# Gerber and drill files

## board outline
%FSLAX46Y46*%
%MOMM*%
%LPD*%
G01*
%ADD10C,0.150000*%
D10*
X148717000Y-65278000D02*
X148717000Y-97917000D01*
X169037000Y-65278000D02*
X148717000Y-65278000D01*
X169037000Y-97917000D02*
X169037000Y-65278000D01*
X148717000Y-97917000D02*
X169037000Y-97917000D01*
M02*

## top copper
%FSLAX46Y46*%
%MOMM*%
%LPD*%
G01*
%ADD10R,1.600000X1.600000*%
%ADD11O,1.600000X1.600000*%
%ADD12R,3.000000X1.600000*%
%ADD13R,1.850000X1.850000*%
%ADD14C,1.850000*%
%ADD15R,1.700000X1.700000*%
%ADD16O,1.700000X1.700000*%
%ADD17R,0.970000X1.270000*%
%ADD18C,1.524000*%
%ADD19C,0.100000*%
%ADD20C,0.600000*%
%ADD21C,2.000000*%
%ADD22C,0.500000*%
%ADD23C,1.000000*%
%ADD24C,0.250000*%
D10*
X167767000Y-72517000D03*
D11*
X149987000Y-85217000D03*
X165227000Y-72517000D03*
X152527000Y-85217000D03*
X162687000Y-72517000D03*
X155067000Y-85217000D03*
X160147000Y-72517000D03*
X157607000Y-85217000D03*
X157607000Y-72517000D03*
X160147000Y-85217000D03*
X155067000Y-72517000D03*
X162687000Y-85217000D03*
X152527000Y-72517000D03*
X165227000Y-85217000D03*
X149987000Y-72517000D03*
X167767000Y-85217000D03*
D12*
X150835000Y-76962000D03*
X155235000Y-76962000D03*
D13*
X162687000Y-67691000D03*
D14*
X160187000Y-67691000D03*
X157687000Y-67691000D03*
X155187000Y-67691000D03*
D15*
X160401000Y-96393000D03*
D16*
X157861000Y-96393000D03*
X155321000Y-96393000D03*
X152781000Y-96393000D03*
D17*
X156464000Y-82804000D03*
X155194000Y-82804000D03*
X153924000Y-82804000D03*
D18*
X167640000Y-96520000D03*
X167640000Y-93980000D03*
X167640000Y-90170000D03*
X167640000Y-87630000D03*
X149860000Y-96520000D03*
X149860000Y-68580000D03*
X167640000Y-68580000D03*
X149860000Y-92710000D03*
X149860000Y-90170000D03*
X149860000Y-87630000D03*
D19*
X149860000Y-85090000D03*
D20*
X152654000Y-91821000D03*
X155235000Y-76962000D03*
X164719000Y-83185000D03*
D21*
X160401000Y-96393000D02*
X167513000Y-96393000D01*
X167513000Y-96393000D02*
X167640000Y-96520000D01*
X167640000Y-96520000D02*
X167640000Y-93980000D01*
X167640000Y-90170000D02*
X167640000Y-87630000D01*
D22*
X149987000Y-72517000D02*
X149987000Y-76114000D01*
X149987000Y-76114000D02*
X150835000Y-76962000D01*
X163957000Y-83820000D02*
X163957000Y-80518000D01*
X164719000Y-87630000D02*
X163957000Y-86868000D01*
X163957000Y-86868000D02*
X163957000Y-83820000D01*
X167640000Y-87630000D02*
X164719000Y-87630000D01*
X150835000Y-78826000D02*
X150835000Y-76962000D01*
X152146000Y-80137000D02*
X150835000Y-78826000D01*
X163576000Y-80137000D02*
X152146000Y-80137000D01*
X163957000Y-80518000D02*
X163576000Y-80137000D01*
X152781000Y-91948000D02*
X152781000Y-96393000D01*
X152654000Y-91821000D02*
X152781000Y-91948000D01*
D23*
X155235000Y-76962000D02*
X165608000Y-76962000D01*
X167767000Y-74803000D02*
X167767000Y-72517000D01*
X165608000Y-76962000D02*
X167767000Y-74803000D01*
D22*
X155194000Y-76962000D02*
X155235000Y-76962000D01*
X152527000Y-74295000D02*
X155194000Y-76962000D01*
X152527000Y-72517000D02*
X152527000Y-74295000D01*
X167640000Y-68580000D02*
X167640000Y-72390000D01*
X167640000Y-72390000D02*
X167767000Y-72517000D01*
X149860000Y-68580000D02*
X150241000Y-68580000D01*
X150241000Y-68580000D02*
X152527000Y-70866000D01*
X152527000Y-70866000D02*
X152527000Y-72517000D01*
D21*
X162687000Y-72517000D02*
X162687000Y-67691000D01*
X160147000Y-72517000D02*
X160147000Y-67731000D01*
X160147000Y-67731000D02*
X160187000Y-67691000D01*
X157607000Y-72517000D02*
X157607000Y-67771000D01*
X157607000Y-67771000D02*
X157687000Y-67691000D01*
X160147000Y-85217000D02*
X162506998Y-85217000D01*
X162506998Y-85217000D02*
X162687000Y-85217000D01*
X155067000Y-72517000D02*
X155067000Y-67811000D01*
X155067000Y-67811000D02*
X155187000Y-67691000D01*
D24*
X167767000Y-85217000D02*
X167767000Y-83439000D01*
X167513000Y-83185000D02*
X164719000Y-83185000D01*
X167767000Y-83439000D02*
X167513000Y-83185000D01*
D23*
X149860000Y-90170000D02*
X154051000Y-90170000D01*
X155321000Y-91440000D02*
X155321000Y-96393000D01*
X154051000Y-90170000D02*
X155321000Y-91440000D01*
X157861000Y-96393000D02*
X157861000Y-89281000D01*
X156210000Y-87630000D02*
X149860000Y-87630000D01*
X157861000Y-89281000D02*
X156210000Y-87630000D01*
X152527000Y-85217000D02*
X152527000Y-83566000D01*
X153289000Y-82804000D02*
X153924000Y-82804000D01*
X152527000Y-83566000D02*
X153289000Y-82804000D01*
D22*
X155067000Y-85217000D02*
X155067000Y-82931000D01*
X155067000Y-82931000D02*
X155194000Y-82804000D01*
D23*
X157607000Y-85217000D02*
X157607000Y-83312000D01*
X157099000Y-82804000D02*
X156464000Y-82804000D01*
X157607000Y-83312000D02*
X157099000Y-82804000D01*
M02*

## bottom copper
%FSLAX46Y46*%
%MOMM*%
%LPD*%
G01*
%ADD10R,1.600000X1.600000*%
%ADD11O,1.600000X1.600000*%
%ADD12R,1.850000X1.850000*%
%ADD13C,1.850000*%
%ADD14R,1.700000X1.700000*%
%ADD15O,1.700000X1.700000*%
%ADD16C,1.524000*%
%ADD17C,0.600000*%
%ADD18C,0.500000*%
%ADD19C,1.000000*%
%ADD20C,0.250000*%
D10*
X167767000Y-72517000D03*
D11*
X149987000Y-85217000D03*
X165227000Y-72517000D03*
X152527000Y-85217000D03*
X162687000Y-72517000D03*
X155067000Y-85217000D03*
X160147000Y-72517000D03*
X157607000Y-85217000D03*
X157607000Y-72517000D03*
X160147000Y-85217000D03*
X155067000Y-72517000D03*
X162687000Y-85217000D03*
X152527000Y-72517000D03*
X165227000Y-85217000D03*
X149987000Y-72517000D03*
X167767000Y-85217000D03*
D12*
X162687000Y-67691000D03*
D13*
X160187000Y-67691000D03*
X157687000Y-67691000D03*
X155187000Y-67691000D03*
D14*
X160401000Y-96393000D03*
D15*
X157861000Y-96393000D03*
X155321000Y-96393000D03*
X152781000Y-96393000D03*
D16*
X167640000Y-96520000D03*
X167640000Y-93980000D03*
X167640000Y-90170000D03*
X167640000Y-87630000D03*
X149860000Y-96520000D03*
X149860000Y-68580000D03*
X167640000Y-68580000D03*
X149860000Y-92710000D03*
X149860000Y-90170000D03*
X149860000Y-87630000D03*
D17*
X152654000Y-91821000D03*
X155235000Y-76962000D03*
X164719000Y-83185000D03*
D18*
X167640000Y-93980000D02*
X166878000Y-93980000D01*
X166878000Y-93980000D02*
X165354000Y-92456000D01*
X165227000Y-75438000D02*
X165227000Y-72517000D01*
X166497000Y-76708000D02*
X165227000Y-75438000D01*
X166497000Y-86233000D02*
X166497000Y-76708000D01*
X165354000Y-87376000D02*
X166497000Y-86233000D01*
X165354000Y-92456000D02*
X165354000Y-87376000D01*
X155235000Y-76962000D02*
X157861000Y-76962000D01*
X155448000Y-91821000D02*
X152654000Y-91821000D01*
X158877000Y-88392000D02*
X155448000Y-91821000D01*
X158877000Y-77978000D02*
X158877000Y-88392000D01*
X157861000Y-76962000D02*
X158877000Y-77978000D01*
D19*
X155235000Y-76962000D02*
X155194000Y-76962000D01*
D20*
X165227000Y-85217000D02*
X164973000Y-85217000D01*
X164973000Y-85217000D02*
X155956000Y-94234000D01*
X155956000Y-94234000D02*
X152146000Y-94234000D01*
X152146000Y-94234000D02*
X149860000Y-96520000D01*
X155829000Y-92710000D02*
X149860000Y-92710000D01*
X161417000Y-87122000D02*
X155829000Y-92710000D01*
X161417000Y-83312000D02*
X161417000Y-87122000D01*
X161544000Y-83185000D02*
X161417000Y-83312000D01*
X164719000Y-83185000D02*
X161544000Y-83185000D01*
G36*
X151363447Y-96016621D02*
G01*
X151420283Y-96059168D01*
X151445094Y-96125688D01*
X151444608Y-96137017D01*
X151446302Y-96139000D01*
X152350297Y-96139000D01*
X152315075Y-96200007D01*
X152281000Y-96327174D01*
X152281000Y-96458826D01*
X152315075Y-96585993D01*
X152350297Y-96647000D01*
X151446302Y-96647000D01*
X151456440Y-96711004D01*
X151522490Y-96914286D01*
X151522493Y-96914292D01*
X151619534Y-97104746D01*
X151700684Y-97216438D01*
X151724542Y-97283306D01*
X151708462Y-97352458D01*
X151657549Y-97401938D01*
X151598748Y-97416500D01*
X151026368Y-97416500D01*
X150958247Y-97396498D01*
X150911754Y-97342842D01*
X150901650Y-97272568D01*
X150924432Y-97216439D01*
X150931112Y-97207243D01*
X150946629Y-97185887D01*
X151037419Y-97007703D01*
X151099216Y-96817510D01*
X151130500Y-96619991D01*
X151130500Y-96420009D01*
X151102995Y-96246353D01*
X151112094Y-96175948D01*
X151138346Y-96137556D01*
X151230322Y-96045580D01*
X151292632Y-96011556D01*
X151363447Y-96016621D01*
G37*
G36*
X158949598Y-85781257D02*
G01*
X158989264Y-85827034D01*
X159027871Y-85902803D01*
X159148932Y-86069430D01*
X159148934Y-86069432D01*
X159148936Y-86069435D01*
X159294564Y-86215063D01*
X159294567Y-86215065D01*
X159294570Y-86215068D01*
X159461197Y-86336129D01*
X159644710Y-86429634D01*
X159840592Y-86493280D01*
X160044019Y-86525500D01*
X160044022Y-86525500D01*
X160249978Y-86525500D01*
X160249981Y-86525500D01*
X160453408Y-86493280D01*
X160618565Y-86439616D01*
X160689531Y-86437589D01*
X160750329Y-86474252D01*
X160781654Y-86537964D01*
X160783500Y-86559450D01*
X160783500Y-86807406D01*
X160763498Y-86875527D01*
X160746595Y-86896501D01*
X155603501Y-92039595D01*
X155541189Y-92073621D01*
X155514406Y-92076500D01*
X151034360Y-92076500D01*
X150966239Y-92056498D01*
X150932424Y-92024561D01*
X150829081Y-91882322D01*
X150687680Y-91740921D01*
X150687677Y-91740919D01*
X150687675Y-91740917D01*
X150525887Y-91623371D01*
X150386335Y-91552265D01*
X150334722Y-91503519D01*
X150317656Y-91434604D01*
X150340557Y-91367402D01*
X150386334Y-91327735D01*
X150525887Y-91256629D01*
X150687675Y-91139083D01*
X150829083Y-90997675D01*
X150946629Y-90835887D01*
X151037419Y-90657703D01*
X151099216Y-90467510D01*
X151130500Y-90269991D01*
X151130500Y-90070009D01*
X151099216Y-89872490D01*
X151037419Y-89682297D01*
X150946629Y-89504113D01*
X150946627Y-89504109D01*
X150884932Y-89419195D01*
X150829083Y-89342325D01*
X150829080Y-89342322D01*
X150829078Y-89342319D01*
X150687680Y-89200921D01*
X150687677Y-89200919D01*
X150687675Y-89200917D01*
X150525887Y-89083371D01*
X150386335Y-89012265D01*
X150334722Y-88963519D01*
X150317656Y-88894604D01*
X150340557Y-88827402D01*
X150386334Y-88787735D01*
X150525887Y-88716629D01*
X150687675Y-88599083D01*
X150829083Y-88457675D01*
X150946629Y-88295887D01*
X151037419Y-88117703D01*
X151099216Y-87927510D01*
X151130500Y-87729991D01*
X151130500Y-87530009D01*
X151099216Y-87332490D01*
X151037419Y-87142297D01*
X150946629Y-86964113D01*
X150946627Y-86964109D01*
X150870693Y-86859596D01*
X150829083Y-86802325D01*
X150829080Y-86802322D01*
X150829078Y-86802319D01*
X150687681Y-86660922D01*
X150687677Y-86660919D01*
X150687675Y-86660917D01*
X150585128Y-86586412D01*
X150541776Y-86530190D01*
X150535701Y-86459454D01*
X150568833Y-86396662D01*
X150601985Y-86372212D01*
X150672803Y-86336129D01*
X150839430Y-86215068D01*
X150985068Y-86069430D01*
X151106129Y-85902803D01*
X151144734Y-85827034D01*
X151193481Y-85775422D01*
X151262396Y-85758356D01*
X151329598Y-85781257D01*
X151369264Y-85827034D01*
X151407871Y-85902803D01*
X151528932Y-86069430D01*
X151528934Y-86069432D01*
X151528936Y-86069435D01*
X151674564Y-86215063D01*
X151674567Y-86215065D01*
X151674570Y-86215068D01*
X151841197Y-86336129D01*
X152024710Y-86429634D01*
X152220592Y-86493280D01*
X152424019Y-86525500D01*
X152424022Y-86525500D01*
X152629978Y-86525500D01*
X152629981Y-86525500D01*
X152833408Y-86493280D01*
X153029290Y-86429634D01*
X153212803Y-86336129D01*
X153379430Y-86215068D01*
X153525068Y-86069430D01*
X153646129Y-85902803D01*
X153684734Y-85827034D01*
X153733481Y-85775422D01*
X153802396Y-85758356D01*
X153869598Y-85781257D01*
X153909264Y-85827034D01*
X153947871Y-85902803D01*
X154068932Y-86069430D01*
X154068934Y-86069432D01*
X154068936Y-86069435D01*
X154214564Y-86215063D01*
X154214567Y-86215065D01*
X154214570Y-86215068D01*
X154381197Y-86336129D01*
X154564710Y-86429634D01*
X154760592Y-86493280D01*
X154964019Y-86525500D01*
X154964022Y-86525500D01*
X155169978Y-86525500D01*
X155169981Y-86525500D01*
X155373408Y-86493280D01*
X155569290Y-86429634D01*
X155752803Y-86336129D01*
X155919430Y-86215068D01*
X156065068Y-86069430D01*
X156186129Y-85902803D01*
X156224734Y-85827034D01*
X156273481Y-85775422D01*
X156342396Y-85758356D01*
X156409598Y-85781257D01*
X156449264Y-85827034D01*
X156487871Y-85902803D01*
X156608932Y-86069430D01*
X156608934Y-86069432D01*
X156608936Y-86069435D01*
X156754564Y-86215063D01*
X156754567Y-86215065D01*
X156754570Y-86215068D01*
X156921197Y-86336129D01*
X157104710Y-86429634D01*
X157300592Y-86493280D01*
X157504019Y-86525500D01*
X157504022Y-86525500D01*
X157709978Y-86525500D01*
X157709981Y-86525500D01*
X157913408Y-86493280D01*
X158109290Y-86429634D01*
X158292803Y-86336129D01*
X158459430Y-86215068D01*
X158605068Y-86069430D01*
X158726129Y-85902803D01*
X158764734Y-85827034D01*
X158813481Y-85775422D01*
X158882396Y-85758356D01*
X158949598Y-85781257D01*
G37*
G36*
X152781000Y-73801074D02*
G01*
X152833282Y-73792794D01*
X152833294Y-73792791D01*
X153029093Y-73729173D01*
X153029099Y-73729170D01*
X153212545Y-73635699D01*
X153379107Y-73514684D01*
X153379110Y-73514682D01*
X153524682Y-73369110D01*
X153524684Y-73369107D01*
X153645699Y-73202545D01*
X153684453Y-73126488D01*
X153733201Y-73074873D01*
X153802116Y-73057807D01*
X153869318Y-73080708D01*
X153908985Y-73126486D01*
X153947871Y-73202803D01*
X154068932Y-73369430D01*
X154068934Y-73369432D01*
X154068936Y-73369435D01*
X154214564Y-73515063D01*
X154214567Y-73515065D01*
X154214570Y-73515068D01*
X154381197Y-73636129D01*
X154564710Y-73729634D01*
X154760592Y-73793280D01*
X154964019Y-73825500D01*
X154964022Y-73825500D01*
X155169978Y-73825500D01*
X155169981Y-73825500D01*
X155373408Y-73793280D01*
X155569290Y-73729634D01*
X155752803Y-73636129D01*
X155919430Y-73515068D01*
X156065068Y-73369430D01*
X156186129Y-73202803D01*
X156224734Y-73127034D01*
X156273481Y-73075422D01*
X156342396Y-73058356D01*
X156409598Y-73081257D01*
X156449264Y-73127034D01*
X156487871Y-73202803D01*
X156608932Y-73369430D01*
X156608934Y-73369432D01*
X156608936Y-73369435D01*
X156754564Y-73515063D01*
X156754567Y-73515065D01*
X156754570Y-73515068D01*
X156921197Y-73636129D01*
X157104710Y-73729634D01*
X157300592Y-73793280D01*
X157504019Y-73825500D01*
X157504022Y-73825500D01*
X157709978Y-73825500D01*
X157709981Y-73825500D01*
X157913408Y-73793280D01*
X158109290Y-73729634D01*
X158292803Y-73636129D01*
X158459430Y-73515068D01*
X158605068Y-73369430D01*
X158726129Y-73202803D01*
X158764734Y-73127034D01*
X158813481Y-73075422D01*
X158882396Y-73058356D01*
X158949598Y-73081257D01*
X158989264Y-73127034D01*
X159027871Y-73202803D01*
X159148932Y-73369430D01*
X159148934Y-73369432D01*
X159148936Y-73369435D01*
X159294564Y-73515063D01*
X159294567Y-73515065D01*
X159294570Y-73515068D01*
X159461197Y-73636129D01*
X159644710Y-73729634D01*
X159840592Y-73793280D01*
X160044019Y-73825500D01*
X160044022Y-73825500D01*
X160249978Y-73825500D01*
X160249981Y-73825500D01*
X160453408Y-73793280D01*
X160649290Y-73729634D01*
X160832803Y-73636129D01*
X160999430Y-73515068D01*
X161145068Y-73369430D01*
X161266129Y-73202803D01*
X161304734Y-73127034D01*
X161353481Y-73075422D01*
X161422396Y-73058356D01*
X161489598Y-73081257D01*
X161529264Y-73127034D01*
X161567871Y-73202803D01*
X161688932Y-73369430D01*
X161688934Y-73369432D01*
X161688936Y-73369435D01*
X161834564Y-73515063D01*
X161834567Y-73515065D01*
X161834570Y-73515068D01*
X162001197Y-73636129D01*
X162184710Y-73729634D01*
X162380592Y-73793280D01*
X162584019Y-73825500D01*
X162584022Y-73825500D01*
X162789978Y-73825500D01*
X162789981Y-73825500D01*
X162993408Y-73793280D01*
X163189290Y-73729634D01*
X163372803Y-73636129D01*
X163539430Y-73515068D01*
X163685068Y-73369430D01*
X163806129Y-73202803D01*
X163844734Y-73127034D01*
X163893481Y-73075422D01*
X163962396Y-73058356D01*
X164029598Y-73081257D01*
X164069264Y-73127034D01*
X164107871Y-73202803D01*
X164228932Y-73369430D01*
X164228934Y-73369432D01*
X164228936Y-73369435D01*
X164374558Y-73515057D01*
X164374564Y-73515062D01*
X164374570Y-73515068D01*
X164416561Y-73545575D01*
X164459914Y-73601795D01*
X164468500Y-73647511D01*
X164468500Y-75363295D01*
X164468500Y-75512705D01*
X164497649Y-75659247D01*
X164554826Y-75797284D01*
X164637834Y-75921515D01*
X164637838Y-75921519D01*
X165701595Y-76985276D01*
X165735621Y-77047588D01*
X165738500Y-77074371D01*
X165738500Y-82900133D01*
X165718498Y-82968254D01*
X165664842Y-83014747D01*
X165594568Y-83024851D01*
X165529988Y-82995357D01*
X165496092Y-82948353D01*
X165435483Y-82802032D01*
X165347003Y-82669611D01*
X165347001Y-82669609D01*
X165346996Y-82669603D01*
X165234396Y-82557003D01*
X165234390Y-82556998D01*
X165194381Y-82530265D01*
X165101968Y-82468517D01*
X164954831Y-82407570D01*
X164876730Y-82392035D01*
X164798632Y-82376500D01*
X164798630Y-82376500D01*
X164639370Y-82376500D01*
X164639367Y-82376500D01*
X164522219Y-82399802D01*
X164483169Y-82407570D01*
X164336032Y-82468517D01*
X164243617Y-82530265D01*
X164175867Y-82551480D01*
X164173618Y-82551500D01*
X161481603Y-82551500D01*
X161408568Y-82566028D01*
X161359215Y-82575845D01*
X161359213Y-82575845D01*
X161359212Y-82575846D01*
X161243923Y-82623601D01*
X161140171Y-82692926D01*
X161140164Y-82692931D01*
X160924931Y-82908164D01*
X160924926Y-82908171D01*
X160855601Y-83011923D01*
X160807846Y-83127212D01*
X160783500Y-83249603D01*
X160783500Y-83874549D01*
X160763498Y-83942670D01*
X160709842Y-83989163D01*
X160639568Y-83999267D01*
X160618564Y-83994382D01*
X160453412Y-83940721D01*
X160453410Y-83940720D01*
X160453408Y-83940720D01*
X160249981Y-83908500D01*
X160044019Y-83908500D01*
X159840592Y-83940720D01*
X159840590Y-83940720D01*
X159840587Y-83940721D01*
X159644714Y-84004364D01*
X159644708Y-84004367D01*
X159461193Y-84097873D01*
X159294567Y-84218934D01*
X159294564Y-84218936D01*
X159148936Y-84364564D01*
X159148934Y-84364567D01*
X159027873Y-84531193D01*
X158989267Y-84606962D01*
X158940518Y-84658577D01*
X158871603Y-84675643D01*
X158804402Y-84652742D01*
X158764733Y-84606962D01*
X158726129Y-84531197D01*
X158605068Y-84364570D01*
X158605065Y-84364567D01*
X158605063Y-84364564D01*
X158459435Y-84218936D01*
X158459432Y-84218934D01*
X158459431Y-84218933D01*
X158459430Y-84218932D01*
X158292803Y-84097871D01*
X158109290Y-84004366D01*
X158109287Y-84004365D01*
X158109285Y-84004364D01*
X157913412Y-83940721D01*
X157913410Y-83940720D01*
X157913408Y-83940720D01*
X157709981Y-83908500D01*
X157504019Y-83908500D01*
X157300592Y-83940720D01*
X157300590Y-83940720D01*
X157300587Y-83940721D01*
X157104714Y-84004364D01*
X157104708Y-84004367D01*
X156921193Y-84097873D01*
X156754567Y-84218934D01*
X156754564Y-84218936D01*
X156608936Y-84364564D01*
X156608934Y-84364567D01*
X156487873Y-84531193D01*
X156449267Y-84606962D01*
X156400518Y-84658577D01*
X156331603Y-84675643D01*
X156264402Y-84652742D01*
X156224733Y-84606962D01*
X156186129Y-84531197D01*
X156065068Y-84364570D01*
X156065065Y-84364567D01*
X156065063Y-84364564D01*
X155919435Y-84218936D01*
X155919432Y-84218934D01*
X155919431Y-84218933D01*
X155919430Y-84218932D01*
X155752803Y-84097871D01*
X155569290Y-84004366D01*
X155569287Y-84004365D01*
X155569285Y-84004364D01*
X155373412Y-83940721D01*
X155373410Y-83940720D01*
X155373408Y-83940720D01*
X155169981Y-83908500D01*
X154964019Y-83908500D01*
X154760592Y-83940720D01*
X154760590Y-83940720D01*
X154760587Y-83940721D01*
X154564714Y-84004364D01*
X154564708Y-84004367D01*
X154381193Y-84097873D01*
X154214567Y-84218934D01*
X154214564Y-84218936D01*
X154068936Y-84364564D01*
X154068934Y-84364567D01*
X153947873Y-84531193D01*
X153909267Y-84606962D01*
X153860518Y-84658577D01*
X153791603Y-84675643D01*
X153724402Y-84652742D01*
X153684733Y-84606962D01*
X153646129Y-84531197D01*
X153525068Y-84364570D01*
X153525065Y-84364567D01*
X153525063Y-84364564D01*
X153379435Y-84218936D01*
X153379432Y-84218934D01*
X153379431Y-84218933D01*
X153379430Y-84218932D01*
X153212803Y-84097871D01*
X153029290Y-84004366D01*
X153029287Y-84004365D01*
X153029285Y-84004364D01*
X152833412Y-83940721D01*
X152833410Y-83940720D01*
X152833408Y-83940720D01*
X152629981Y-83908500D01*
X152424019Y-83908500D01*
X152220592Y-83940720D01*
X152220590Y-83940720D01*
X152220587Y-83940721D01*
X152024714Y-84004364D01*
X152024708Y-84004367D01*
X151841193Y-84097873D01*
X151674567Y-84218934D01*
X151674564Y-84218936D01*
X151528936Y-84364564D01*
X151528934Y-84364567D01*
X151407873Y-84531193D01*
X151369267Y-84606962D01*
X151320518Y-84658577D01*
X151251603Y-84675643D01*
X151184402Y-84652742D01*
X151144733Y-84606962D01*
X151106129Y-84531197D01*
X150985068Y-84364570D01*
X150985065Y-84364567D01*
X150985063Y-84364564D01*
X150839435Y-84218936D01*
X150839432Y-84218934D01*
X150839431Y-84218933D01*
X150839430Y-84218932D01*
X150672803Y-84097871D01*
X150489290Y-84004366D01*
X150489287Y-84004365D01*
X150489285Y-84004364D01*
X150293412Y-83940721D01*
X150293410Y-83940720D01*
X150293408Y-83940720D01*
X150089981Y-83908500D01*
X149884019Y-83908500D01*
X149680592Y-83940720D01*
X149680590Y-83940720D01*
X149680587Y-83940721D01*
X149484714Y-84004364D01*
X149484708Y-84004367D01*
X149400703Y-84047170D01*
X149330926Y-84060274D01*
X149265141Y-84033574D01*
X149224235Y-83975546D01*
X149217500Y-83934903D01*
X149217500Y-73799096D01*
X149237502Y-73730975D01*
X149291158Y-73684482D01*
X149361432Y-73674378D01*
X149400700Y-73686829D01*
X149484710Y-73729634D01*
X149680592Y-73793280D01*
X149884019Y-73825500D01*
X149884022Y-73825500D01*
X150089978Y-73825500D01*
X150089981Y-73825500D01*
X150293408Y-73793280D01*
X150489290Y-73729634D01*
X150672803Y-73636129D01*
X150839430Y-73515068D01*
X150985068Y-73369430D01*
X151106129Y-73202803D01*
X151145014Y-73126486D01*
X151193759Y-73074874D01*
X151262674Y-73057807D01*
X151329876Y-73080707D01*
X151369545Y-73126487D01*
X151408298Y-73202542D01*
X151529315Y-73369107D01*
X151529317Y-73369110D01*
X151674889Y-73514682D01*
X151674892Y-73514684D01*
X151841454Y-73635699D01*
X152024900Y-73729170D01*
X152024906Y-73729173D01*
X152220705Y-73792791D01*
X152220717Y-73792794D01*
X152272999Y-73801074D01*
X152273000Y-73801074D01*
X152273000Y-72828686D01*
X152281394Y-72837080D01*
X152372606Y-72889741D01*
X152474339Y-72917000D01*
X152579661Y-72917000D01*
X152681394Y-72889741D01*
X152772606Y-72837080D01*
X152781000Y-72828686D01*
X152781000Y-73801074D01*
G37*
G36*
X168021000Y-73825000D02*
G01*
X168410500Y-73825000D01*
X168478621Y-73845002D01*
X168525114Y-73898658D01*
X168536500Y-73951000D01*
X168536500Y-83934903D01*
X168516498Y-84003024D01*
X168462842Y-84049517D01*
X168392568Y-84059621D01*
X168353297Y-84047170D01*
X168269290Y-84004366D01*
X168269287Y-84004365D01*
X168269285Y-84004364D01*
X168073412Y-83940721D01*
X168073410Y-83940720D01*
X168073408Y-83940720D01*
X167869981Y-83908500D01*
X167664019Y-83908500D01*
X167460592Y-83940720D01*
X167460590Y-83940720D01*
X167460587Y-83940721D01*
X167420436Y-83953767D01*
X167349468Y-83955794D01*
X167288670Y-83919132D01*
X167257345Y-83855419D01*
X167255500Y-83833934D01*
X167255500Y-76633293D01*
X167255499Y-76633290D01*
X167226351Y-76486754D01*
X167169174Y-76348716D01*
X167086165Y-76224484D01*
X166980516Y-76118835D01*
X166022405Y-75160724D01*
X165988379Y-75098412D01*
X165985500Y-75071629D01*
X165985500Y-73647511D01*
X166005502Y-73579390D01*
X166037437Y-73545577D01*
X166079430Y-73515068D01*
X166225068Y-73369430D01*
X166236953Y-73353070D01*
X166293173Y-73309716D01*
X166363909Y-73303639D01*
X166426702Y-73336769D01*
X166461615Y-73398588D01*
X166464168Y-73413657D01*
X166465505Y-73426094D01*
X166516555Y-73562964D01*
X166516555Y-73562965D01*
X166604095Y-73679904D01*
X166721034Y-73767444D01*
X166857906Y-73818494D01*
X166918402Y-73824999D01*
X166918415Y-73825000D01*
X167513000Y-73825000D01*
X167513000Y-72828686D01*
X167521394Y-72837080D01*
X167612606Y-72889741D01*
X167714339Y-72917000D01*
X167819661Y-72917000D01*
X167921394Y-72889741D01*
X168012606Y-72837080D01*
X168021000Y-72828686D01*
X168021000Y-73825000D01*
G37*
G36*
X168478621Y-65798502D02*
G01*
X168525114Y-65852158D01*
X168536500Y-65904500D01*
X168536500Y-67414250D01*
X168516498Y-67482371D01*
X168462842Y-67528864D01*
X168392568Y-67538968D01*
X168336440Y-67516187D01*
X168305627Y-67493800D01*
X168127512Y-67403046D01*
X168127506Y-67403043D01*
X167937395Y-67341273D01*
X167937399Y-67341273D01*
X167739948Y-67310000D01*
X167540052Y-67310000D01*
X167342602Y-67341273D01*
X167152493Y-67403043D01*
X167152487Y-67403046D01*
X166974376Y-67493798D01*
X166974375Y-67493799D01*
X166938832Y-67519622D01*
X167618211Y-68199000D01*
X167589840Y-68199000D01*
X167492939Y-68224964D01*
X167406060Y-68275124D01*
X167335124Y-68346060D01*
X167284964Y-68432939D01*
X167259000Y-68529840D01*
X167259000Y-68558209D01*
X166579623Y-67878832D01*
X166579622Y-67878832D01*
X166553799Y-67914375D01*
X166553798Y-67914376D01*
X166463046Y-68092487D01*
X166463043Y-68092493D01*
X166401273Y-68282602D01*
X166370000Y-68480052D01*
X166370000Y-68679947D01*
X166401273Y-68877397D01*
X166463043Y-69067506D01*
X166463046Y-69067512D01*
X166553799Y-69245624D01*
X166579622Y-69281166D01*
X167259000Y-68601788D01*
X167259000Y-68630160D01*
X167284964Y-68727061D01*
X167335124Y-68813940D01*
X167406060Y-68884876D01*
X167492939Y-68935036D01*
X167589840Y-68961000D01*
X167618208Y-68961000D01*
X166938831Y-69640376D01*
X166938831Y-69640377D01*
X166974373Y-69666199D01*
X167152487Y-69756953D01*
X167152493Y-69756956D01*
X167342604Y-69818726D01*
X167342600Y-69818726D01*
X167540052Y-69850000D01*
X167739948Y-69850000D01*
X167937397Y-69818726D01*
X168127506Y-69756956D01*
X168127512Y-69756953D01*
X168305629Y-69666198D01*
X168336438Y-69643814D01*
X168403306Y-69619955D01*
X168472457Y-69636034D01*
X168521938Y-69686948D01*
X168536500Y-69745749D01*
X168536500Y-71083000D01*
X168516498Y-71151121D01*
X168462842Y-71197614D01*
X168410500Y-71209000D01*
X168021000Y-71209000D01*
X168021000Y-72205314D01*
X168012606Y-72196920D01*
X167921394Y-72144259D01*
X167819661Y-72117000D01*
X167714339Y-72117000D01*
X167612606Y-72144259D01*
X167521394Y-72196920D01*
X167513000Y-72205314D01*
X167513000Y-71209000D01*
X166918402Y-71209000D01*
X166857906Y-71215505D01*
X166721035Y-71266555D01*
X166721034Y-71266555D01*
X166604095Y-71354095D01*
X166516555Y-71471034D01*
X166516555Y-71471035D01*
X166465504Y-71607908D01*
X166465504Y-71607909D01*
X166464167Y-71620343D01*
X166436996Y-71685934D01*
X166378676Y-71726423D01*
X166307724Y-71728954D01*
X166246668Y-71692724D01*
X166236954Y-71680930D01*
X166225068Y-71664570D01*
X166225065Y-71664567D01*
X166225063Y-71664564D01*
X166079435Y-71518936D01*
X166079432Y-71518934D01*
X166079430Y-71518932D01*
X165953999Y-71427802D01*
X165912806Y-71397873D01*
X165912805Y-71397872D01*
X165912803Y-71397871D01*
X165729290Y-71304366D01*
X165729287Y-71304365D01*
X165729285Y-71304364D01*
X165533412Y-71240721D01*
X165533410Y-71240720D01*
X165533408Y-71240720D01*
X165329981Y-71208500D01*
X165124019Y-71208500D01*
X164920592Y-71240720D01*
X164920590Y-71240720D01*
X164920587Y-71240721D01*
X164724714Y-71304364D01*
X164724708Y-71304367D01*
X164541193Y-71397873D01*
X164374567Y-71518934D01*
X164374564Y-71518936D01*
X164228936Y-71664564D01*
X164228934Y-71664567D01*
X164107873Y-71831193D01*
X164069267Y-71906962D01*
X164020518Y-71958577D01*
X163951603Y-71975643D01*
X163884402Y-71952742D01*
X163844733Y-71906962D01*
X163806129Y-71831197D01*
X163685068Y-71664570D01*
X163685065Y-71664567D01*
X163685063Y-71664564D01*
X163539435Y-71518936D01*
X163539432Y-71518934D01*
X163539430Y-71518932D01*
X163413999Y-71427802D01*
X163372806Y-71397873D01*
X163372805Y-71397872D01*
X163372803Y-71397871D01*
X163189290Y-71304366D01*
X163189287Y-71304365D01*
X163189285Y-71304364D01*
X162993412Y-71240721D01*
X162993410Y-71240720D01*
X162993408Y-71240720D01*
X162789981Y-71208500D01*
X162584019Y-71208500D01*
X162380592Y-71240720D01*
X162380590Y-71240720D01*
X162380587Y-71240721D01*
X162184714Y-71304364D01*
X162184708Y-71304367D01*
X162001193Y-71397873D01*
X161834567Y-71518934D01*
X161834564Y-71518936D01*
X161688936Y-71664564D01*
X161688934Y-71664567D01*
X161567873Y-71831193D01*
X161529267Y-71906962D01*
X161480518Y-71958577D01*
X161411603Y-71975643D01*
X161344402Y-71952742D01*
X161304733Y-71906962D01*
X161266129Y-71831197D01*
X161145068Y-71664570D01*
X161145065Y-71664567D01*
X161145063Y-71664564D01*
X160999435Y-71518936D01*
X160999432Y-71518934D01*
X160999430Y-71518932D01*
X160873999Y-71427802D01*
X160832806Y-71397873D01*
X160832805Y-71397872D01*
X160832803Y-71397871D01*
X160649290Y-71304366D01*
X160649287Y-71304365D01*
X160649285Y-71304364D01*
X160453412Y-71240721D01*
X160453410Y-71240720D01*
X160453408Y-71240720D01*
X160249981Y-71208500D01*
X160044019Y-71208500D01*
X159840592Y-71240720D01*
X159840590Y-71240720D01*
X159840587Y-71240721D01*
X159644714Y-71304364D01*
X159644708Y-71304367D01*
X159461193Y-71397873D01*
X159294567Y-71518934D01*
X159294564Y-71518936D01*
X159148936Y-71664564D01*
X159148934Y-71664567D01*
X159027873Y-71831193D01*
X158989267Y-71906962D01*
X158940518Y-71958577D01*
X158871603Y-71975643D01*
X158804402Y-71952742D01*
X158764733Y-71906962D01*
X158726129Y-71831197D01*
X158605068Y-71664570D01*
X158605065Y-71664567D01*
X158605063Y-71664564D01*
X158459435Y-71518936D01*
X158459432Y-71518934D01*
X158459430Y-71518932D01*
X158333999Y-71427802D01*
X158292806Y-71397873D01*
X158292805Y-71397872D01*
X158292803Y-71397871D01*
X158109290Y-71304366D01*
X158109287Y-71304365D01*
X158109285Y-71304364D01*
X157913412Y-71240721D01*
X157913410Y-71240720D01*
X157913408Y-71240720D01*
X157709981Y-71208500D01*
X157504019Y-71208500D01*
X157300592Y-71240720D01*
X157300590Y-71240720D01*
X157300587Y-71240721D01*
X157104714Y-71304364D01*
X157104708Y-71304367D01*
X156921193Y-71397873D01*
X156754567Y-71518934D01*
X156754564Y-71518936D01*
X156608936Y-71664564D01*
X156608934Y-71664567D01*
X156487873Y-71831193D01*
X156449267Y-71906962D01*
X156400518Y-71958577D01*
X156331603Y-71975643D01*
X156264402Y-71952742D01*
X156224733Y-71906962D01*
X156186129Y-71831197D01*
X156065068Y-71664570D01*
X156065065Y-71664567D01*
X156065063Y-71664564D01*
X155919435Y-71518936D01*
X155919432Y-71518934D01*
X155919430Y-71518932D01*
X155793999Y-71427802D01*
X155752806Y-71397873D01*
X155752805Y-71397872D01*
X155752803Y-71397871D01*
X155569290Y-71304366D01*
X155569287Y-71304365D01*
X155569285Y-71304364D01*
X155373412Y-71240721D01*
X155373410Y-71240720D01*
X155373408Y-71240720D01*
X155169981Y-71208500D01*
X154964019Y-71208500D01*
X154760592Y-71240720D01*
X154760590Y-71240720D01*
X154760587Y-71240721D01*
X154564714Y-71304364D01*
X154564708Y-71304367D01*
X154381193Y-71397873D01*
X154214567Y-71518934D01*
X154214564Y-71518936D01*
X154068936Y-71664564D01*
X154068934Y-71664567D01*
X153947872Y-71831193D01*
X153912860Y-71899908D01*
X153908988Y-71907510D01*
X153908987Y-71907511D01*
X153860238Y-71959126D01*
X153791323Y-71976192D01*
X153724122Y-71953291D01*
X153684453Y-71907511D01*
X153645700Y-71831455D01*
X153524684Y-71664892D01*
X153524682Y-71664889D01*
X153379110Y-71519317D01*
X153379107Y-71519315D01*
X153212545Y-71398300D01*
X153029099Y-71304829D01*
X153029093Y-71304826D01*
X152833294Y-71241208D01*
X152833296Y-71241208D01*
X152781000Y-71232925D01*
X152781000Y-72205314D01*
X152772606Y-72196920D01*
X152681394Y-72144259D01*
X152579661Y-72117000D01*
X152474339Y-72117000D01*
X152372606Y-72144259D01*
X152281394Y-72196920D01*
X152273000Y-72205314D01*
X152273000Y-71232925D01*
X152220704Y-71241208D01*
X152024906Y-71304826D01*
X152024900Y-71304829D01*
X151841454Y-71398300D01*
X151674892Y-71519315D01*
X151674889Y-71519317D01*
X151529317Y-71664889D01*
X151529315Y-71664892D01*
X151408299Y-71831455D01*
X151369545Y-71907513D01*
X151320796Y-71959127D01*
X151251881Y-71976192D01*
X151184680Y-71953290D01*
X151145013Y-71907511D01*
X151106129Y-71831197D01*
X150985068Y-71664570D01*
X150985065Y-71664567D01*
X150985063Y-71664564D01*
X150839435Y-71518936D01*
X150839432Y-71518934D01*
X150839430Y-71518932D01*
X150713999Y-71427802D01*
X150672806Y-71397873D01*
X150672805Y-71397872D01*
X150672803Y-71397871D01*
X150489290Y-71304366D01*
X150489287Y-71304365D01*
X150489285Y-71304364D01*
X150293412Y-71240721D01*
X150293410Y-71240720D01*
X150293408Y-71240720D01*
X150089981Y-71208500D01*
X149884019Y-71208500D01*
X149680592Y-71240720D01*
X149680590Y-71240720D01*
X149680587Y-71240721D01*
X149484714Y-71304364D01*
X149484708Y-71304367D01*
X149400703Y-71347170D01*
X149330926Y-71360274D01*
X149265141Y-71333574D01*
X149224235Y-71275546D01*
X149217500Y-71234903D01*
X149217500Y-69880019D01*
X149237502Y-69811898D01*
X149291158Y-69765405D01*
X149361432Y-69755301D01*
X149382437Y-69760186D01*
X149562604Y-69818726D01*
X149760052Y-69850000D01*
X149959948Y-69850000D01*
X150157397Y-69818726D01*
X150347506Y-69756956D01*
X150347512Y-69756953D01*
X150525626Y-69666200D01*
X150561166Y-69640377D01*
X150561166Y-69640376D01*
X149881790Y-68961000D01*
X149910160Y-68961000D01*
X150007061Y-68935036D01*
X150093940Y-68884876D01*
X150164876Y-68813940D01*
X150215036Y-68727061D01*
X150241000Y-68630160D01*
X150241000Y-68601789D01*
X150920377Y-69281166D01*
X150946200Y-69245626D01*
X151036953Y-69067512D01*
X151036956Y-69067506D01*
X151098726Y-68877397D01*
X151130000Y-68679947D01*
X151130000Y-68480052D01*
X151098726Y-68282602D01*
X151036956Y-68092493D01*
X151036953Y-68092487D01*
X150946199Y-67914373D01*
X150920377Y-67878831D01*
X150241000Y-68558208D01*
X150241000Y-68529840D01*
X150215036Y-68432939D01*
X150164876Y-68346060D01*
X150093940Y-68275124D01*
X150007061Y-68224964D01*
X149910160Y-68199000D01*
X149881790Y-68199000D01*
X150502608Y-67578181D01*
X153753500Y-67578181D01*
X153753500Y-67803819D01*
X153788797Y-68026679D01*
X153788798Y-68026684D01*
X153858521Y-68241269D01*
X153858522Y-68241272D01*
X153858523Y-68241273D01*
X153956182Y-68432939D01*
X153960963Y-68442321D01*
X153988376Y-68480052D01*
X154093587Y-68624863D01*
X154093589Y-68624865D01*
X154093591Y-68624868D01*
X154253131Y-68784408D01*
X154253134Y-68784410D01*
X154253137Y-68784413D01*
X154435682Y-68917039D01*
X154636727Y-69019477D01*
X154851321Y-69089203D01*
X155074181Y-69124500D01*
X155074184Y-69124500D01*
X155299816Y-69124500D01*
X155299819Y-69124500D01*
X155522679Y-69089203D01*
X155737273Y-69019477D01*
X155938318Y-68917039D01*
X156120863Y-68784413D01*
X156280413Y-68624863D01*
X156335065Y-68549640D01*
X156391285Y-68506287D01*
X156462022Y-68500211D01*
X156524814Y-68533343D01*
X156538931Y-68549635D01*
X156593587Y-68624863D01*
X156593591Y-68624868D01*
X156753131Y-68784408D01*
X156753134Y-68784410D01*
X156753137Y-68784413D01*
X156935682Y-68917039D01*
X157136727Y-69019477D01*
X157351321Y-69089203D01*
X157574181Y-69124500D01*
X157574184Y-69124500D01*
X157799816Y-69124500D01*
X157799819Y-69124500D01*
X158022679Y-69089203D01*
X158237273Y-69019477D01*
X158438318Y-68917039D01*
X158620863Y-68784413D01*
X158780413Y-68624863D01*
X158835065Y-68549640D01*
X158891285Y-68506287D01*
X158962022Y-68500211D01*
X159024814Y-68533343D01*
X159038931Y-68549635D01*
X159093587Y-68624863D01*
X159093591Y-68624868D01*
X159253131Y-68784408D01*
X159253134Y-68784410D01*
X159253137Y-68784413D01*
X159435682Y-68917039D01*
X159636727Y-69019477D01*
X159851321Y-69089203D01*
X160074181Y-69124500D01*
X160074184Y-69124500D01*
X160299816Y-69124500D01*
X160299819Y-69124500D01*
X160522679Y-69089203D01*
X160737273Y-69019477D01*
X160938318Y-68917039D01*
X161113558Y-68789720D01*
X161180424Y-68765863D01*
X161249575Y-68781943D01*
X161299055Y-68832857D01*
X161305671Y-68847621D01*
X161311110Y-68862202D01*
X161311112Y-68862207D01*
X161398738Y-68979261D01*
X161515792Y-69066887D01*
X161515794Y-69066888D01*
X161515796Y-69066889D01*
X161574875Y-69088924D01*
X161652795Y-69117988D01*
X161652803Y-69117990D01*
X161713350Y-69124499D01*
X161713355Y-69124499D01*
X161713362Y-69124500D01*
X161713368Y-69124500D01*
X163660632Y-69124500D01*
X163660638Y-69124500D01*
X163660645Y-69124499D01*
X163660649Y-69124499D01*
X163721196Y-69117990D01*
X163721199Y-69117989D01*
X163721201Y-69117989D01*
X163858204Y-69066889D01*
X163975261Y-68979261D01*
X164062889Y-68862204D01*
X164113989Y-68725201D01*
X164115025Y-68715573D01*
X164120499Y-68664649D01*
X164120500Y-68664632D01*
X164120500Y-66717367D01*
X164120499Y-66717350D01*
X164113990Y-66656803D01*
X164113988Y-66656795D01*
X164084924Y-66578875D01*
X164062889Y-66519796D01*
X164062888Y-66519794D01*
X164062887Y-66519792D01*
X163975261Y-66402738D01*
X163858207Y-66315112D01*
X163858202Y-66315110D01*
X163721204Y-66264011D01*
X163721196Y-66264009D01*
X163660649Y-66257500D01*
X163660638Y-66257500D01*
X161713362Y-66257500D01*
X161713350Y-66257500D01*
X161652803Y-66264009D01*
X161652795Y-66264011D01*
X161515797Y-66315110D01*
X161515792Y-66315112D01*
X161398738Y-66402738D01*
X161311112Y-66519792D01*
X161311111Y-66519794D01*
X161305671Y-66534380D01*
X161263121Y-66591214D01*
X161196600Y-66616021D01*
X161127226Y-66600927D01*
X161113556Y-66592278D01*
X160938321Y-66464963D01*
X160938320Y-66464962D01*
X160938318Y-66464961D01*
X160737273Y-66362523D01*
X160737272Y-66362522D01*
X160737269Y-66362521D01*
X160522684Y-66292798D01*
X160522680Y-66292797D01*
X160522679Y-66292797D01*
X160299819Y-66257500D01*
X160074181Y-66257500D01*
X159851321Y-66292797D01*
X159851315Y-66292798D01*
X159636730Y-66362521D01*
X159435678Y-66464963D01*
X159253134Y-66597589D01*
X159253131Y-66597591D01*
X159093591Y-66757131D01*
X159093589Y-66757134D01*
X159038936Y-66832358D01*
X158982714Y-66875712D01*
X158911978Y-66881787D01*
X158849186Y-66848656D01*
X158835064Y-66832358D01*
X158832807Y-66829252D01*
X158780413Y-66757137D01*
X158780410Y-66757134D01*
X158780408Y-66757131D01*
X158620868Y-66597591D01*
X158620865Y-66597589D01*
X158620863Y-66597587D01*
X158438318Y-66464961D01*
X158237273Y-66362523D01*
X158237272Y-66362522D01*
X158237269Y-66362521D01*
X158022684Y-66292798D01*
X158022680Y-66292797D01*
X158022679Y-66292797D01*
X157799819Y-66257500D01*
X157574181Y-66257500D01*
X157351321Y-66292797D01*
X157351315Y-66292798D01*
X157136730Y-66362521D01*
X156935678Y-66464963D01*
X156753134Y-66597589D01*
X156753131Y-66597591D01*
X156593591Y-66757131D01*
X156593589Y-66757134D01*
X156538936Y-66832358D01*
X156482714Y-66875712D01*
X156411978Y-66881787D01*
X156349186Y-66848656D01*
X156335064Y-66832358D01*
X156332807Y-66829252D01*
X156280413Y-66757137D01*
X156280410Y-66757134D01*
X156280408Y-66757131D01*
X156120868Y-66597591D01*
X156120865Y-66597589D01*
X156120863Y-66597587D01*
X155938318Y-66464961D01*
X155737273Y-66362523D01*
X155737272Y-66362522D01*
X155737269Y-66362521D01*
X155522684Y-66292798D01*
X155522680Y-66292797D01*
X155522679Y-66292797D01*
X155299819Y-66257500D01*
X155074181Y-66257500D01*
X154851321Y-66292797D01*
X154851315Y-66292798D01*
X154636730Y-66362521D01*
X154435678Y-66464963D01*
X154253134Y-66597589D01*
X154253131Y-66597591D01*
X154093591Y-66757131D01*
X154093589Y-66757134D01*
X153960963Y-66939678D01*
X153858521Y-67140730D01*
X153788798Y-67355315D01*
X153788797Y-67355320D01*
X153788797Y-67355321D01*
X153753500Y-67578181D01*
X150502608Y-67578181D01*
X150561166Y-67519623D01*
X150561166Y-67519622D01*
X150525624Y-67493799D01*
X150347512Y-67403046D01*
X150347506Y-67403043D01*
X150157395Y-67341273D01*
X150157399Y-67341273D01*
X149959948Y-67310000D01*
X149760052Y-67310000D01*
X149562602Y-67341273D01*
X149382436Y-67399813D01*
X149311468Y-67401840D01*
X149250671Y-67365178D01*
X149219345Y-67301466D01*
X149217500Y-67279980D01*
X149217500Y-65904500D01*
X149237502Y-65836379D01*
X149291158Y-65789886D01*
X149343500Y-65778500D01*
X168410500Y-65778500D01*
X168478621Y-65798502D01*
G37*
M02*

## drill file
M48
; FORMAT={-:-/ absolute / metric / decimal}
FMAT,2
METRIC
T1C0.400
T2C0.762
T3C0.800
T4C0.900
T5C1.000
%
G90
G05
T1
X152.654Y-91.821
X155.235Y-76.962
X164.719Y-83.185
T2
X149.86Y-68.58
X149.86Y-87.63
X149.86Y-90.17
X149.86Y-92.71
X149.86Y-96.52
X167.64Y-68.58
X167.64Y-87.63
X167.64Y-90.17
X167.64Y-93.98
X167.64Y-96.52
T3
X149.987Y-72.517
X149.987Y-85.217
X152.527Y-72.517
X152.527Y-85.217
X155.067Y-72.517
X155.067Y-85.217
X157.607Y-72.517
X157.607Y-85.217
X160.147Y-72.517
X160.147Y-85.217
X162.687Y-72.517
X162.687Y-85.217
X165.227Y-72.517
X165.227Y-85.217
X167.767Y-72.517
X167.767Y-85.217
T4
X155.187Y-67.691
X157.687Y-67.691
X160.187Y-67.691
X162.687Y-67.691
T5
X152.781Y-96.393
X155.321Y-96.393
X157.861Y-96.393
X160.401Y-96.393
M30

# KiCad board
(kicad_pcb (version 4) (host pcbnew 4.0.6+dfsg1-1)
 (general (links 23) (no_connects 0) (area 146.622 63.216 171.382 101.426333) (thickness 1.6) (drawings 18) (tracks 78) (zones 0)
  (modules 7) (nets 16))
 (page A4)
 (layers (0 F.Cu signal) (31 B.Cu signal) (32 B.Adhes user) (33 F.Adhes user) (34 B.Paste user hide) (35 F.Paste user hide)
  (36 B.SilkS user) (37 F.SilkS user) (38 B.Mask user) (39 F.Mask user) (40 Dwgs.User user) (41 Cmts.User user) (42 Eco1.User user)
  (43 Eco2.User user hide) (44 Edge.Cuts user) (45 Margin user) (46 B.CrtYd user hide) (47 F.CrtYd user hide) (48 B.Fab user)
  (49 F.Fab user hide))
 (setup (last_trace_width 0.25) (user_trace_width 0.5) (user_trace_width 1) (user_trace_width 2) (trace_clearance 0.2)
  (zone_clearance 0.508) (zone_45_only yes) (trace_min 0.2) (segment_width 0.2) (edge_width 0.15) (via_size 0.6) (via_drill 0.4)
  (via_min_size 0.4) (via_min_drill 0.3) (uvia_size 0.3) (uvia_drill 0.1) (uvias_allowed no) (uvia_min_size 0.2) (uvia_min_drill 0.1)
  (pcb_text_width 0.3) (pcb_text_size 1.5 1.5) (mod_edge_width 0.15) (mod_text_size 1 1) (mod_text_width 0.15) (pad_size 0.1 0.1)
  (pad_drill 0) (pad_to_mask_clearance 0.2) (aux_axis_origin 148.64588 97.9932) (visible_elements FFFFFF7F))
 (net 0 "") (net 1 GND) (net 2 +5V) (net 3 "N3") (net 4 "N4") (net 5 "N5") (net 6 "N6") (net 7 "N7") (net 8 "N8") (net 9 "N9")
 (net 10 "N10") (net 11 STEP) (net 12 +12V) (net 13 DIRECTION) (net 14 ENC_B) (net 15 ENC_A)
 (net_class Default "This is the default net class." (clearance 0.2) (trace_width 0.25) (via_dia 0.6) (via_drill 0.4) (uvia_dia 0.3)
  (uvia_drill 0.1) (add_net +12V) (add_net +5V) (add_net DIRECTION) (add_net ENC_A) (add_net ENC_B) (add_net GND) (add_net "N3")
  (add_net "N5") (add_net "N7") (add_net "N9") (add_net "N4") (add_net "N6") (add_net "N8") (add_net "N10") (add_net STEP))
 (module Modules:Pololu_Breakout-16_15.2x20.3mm (layer F.Cu) (at 167.767 72.517 270)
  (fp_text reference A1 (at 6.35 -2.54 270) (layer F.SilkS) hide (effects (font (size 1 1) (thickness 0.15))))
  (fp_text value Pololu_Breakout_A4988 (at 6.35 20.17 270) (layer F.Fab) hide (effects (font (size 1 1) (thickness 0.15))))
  (pad 1 thru_hole rect (at 0 0 270) (size 1.6 1.6) (drill 0.8) (layers *.Cu *.Mask) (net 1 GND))
  (pad 9 thru_hole oval (at 12.7 17.78 270) (size 1.6 1.6) (drill 0.8) (layers *.Cu *.Mask))
  (pad 2 thru_hole oval (at 0 2.54 270) (size 1.6 1.6) (drill 0.8) (layers *.Cu *.Mask) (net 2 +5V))
  (pad 10 thru_hole oval (at 12.7 15.24 270) (size 1.6 1.6) (drill 0.8) (layers *.Cu *.Mask) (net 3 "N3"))
  (pad 3 thru_hole oval (at 0 5.08 270) (size 1.6 1.6) (drill 0.8) (layers *.Cu *.Mask) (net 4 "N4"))
  (pad 11 thru_hole oval (at 12.7 12.7 270) (size 1.6 1.6) (drill 0.8) (layers *.Cu *.Mask) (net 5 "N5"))
  (pad 4 thru_hole oval (at 0 7.62 270) (size 1.6 1.6) (drill 0.8) (layers *.Cu *.Mask) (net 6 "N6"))
  (pad 12 thru_hole oval (at 12.7 10.16 270) (size 1.6 1.6) (drill 0.8) (layers *.Cu *.Mask) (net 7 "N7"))
  (pad 5 thru_hole oval (at 0 10.16 270) (size 1.6 1.6) (drill 0.8) (layers *.Cu *.Mask) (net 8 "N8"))
  (pad 13 thru_hole oval (at 12.7 7.62 270) (size 1.6 1.6) (drill 0.8) (layers *.Cu *.Mask) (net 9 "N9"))
  (pad 6 thru_hole oval (at 0 12.7 270) (size 1.6 1.6) (drill 0.8) (layers *.Cu *.Mask) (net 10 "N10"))
  (pad 14 thru_hole oval (at 12.7 5.08 270) (size 1.6 1.6) (drill 0.8) (layers *.Cu *.Mask) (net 9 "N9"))
  (pad 7 thru_hole oval (at 0 15.24 270) (size 1.6 1.6) (drill 0.8) (layers *.Cu *.Mask) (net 1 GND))
  (pad 15 thru_hole oval (at 12.7 2.54 270) (size 1.6 1.6) (drill 0.8) (layers *.Cu *.Mask) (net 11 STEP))
  (pad 8 thru_hole oval (at 0 17.78 270) (size 1.6 1.6) (drill 0.8) (layers *.Cu *.Mask) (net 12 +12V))
  (pad 16 thru_hole oval (at 12.7 0 270) (size 1.6 1.6) (drill 0.8) (layers *.Cu *.Mask) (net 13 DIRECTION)))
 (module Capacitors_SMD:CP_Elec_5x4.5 (layer F.Cu) (at 153.035 76.962)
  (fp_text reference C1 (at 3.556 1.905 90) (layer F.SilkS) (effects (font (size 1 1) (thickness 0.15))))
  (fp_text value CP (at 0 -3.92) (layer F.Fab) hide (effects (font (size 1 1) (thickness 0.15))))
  (pad 1 smd rect (at -2.2 0 180) (size 3 1.6) (layers F.Cu F.Paste F.Mask) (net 12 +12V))
  (pad 2 smd rect (at 2.2 0 180) (size 3 1.6) (layers F.Cu F.Paste F.Mask) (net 1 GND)))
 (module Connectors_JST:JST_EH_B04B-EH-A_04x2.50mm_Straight (layer F.Cu) (at 162.687 67.691 180)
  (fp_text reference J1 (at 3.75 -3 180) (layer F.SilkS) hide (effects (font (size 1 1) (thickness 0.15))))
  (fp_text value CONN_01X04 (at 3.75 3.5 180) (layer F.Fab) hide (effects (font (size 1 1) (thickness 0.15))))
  (pad 1 thru_hole rect (at 0 0 180) (size 1.85 1.85) (drill 0.9) (layers *.Cu *.Mask) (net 4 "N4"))
  (pad 2 thru_hole circle (at 2.5 0 180) (size 1.85 1.85) (drill 0.9) (layers *.Cu *.Mask) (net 6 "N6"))
  (pad 3 thru_hole circle (at 5 0 180) (size 1.85 1.85) (drill 0.9) (layers *.Cu *.Mask) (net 8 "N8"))
  (pad 4 thru_hole circle (at 7.5 0 180) (size 1.85 1.85) (drill 0.9) (layers *.Cu *.Mask) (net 10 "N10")))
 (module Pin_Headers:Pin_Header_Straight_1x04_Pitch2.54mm (layer F.Cu) (at 160.401 96.393 270)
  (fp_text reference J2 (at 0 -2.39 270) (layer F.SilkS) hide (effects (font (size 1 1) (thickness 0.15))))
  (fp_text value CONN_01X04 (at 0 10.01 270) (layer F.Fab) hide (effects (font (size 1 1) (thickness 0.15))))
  (pad 1 thru_hole rect (at 0 0 270) (size 1.7 1.7) (drill 1) (layers *.Cu *.Mask) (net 2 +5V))
  (pad 2 thru_hole oval (at 0 2.54 270) (size 1.7 1.7) (drill 1) (layers *.Cu *.Mask) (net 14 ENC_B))
  (pad 3 thru_hole oval (at 0 5.08 270) (size 1.7 1.7) (drill 1) (layers *.Cu *.Mask) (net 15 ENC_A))
  (pad 4 thru_hole oval (at 0 7.62 270) (size 1.7 1.7) (drill 1) (layers *.Cu *.Mask) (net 1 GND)))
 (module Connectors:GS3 (layer F.Cu) (at 155.194 82.804 270)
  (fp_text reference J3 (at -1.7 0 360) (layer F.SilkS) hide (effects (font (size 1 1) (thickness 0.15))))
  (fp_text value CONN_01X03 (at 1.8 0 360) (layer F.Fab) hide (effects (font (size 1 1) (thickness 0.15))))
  (pad 1 smd rect (at 0 -1.27 270) (size 1.27 0.97) (layers F.Cu F.Paste F.Mask) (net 7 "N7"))
  (pad 2 smd rect (at 0 0 270) (size 1.27 0.97) (layers F.Cu F.Paste F.Mask) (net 5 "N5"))
  (pad 3 smd rect (at 0 1.27 270) (size 1.27 0.97) (layers F.Cu F.Paste F.Mask) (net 3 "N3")))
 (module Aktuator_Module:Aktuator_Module (layer F.Cu) (at 148.59 97.79)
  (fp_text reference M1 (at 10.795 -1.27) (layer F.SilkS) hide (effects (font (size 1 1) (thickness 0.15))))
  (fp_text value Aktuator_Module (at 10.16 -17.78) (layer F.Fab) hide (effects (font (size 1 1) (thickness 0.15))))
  (pad 1 thru_hole circle (at 19.05 -1.27) (size 1.524 1.524) (drill 0.762) (layers *.Cu *.Mask) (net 2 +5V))
  (pad 1 thru_hole circle (at 19.05 -3.81) (size 1.524 1.524) (drill 0.762) (layers *.Cu *.Mask) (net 2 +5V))
  (pad 2 thru_hole circle (at 19.05 -7.62) (size 1.524 1.524) (drill 0.762) (layers *.Cu *.Mask) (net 12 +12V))
  (pad 2 thru_hole circle (at 19.05 -10.16) (size 1.524 1.524) (drill 0.762) (layers *.Cu *.Mask) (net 12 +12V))
  (pad 3 thru_hole circle (at 1.27 -1.27) (size 1.524 1.524) (drill 0.762) (layers *.Cu *.Mask) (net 11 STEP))
  (pad 4 thru_hole circle (at 1.27 -29.21) (size 1.524 1.524) (drill 0.762) (layers *.Cu *.Mask) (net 1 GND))
  (pad 4 thru_hole circle (at 19.05 -29.21) (size 1.524 1.524) (drill 0.762) (layers *.Cu *.Mask) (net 1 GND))
  (pad 6 thru_hole circle (at 1.27 -5.08) (size 1.524 1.524) (drill 0.762) (layers *.Cu *.Mask) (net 13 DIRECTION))
  (pad 7 thru_hole circle (at 1.27 -7.62) (size 1.524 1.524) (drill 0.762) (layers *.Cu *.Mask) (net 15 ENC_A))
  (pad 8 thru_hole circle (at 1.27 -10.16) (size 1.524 1.524) (drill 0.762) (layers *.Cu *.Mask) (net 14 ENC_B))
  (pad 9 smd circle (at 1.27 -12.7) (size 0.1 0.1) (layers F.Cu F.Paste F.Mask)))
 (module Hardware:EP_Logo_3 (layer F.Cu) (at 162.56 78.359)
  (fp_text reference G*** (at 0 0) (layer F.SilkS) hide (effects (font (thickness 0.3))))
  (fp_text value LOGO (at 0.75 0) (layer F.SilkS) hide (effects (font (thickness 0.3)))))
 (gr_line (start 148.717 65.278) (end 148.717 97.917) (angle 90) (layer Edge.Cuts) (width 0.15))
 (gr_line (start 169.037 65.278) (end 148.717 65.278) (angle 90) (layer Edge.Cuts) (width 0.15))
 (gr_line (start 169.037 97.917) (end 169.037 65.278) (angle 90) (layer Edge.Cuts) (width 0.15))
 (gr_line (start 148.717 97.917) (end 169.037 97.917) (angle 90) (layer Edge.Cuts) (width 0.15))
 (segment (start 167.64 93.98) (end 166.878 93.98) (width 0.5) (layer B.Cu) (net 2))
 (segment (start 166.878 93.98) (end 165.354 92.456) (width 0.5) (layer B.Cu) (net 2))
 (segment (start 165.227 75.438) (end 165.227 72.517) (width 0.5) (layer B.Cu) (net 2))
 (segment (start 166.497 76.708) (end 165.227 75.438) (width 0.5) (layer B.Cu) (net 2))
 (segment (start 166.497 86.233) (end 166.497 76.708) (width 0.5) (layer B.Cu) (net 2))
 (segment (start 165.354 87.376) (end 166.497 86.233) (width 0.5) (layer B.Cu) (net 2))
 (segment (start 165.354 92.456) (end 165.354 87.376) (width 0.5) (layer B.Cu) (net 2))
 (segment (start 160.401 96.393) (end 167.513 96.393) (width 2) (layer F.Cu) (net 2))
 (segment (start 167.513 96.393) (end 167.64 96.52) (width 2) (layer F.Cu) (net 2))
 (segment (start 167.64 96.52) (end 167.64 93.98) (width 2) (layer F.Cu) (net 2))
 (segment (start 167.64 90.17) (end 167.64 87.63) (width 2) (layer F.Cu) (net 12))
 (segment (start 149.987 72.517) (end 149.987 76.114) (width 0.5) (layer F.Cu) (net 12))
 (segment (start 149.987 76.114) (end 150.835 76.962) (width 0.5) (layer F.Cu) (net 12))
 (segment (start 163.957 83.82) (end 163.957 80.518) (width 0.5) (layer F.Cu) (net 12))
 (segment (start 164.719 87.63) (end 163.957 86.868) (width 0.5) (layer F.Cu) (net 12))
 (segment (start 163.957 86.868) (end 163.957 83.82) (width 0.5) (layer F.Cu) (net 12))
 (segment (start 167.64 87.63) (end 164.719 87.63) (width 0.5) (layer F.Cu) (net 12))
 (segment (start 150.835 78.826) (end 150.835 76.962) (width 0.5) (layer F.Cu) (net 12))
 (segment (start 152.146 80.137) (end 150.835 78.826) (width 0.5) (layer F.Cu) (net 12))
 (segment (start 163.576 80.137) (end 152.146 80.137) (width 0.5) (layer F.Cu) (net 12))
 (segment (start 163.957 80.518) (end 163.576 80.137) (width 0.5) (layer F.Cu) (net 12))
 (segment (start 155.235 76.962) (end 157.861 76.962) (width 0.5) (layer B.Cu) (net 1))
 (segment (start 152.781 91.948) (end 152.781 96.393) (width 0.5) (layer F.Cu) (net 1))
 (segment (start 152.654 91.821) (end 152.781 91.948) (width 0.5) (layer F.Cu) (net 1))
 (via (at 152.654 91.821) (size 0.6) (drill 0.4) (layers F.Cu B.Cu) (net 1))
 (segment (start 155.448 91.821) (end 152.654 91.821) (width 0.5) (layer B.Cu) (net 1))
 (segment (start 158.877 88.392) (end 155.448 91.821) (width 0.5) (layer B.Cu) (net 1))
 (segment (start 158.877 77.978) (end 158.877 88.392) (width 0.5) (layer B.Cu) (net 1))
 (segment (start 157.861 76.962) (end 158.877 77.978) (width 0.5) (layer B.Cu) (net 1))
 (segment (start 155.235 76.962) (end 165.608 76.962) (width 1) (layer F.Cu) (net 1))
 (segment (start 167.767 74.803) (end 167.767 72.517) (width 1) (layer F.Cu) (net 1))
 (segment (start 165.608 76.962) (end 167.767 74.803) (width 1) (layer F.Cu) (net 1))
 (via (at 155.235 76.962) (size 0.6) (drill 0.4) (layers F.Cu B.Cu) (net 1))
 (segment (start 155.194 76.962) (end 155.235 76.962) (width 0.5) (layer F.Cu) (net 1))
 (segment (start 152.527 74.295) (end 155.194 76.962) (width 0.5) (layer F.Cu) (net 1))
 (segment (start 152.527 72.517) (end 152.527 74.295) (width 0.5) (layer F.Cu) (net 1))
 (segment (start 155.235 76.962) (end 155.194 76.962) (width 1) (layer B.Cu) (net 1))
 (segment (start 167.64 68.58) (end 167.64 72.39) (width 0.5) (layer F.Cu) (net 1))
 (segment (start 167.64 72.39) (end 167.767 72.517) (width 0.5) (layer F.Cu) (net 1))
 (segment (start 149.86 68.58) (end 150.241 68.58) (width 0.5) (layer F.Cu) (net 1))
 (segment (start 150.241 68.58) (end 152.527 70.866) (width 0.5) (layer F.Cu) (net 1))
 (segment (start 152.527 70.866) (end 152.527 72.517) (width 0.5) (layer F.Cu) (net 1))
 (segment (start 162.687 72.517) (end 162.687 67.691) (width 2) (layer F.Cu) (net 4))
 (segment (start 160.147 72.517) (end 160.147 67.731) (width 2) (layer F.Cu) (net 6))
 (segment (start 160.147 67.731) (end 160.187 67.691) (width 2) (layer F.Cu) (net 6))
 (segment (start 157.607 72.517) (end 157.607 67.771) (width 2) (layer F.Cu) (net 8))
 (segment (start 157.607 67.771) (end 157.687 67.691) (width 2) (layer F.Cu) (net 8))
 (segment (start 160.147 85.217) (end 162.506998 85.217) (width 2) (layer F.Cu) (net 9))
 (segment (start 162.506998 85.217) (end 162.687 85.217) (width 2) (layer F.Cu) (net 9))
 (segment (start 155.067 72.517) (end 155.067 67.811) (width 2) (layer F.Cu) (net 10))
 (segment (start 155.067 67.811) (end 155.187 67.691) (width 2) (layer F.Cu) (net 10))
 (segment (start 165.227 85.217) (end 164.973 85.217) (width 0.25) (layer B.Cu) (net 11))
 (segment (start 164.973 85.217) (end 155.956 94.234) (width 0.25) (layer B.Cu) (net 11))
 (segment (start 155.956 94.234) (end 152.146 94.234) (width 0.25) (layer B.Cu) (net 11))
 (segment (start 152.146 94.234) (end 149.86 96.52) (width 0.25) (layer B.Cu) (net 11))
 (segment (start 167.767 85.217) (end 167.767 83.439) (width 0.25) (layer F.Cu) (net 13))
 (segment (start 155.829 92.71) (end 149.86 92.71) (width 0.25) (layer B.Cu) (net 13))
 (segment (start 161.417 87.122) (end 155.829 92.71) (width 0.25) (layer B.Cu) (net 13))
 (segment (start 161.417 83.312) (end 161.417 87.122) (width 0.25) (layer B.Cu) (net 13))
 (segment (start 161.544 83.185) (end 161.417 83.312) (width 0.25) (layer B.Cu) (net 13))
 (segment (start 164.719 83.185) (end 161.544 83.185) (width 0.25) (layer B.Cu) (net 13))
 (via (at 164.719 83.185) (size 0.6) (drill 0.4) (layers F.Cu B.Cu) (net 13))
 (segment (start 167.513 83.185) (end 164.719 83.185) (width 0.25) (layer F.Cu) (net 13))
 (segment (start 167.767 83.439) (end 167.513 83.185) (width 0.25) (layer F.Cu) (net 13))
 (segment (start 149.86 90.17) (end 154.051 90.17) (width 1) (layer F.Cu) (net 15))
 (segment (start 155.321 91.44) (end 155.321 96.393) (width 1) (layer F.Cu) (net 15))
 (segment (start 154.051 90.17) (end 155.321 91.44) (width 1) (layer F.Cu) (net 15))
 (segment (start 157.861 96.393) (end 157.861 89.281) (width 1) (layer F.Cu) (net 14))
 (segment (start 156.21 87.63) (end 149.86 87.63) (width 1) (layer F.Cu) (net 14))
 (segment (start 157.861 89.281) (end 156.21 87.63) (width 1) (layer F.Cu) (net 14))
 (segment (start 152.527 85.217) (end 152.527 83.566) (width 1) (layer F.Cu) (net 3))
 (segment (start 153.289 82.804) (end 153.924 82.804) (width 1) (layer F.Cu) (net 3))
 (segment (start 152.527 83.566) (end 153.289 82.804) (width 1) (layer F.Cu) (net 3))
 (segment (start 155.067 85.217) (end 155.067 82.931) (width 0.5) (layer F.Cu) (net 5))
 (segment (start 155.067 82.931) (end 155.194 82.804) (width 0.5) (layer F.Cu) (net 5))
 (segment (start 157.607 85.217) (end 157.607 83.312) (width 1) (layer F.Cu) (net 7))
 (segment (start 157.099 82.804) (end 156.464 82.804) (width 1) (layer F.Cu) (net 7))
 (segment (start 157.607 83.312) (end 157.099 82.804) (width 1) (layer F.Cu) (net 7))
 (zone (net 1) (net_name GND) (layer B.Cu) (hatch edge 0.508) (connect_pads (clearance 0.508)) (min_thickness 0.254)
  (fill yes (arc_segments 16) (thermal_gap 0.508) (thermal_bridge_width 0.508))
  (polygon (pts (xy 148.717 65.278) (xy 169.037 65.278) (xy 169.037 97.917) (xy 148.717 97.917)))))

